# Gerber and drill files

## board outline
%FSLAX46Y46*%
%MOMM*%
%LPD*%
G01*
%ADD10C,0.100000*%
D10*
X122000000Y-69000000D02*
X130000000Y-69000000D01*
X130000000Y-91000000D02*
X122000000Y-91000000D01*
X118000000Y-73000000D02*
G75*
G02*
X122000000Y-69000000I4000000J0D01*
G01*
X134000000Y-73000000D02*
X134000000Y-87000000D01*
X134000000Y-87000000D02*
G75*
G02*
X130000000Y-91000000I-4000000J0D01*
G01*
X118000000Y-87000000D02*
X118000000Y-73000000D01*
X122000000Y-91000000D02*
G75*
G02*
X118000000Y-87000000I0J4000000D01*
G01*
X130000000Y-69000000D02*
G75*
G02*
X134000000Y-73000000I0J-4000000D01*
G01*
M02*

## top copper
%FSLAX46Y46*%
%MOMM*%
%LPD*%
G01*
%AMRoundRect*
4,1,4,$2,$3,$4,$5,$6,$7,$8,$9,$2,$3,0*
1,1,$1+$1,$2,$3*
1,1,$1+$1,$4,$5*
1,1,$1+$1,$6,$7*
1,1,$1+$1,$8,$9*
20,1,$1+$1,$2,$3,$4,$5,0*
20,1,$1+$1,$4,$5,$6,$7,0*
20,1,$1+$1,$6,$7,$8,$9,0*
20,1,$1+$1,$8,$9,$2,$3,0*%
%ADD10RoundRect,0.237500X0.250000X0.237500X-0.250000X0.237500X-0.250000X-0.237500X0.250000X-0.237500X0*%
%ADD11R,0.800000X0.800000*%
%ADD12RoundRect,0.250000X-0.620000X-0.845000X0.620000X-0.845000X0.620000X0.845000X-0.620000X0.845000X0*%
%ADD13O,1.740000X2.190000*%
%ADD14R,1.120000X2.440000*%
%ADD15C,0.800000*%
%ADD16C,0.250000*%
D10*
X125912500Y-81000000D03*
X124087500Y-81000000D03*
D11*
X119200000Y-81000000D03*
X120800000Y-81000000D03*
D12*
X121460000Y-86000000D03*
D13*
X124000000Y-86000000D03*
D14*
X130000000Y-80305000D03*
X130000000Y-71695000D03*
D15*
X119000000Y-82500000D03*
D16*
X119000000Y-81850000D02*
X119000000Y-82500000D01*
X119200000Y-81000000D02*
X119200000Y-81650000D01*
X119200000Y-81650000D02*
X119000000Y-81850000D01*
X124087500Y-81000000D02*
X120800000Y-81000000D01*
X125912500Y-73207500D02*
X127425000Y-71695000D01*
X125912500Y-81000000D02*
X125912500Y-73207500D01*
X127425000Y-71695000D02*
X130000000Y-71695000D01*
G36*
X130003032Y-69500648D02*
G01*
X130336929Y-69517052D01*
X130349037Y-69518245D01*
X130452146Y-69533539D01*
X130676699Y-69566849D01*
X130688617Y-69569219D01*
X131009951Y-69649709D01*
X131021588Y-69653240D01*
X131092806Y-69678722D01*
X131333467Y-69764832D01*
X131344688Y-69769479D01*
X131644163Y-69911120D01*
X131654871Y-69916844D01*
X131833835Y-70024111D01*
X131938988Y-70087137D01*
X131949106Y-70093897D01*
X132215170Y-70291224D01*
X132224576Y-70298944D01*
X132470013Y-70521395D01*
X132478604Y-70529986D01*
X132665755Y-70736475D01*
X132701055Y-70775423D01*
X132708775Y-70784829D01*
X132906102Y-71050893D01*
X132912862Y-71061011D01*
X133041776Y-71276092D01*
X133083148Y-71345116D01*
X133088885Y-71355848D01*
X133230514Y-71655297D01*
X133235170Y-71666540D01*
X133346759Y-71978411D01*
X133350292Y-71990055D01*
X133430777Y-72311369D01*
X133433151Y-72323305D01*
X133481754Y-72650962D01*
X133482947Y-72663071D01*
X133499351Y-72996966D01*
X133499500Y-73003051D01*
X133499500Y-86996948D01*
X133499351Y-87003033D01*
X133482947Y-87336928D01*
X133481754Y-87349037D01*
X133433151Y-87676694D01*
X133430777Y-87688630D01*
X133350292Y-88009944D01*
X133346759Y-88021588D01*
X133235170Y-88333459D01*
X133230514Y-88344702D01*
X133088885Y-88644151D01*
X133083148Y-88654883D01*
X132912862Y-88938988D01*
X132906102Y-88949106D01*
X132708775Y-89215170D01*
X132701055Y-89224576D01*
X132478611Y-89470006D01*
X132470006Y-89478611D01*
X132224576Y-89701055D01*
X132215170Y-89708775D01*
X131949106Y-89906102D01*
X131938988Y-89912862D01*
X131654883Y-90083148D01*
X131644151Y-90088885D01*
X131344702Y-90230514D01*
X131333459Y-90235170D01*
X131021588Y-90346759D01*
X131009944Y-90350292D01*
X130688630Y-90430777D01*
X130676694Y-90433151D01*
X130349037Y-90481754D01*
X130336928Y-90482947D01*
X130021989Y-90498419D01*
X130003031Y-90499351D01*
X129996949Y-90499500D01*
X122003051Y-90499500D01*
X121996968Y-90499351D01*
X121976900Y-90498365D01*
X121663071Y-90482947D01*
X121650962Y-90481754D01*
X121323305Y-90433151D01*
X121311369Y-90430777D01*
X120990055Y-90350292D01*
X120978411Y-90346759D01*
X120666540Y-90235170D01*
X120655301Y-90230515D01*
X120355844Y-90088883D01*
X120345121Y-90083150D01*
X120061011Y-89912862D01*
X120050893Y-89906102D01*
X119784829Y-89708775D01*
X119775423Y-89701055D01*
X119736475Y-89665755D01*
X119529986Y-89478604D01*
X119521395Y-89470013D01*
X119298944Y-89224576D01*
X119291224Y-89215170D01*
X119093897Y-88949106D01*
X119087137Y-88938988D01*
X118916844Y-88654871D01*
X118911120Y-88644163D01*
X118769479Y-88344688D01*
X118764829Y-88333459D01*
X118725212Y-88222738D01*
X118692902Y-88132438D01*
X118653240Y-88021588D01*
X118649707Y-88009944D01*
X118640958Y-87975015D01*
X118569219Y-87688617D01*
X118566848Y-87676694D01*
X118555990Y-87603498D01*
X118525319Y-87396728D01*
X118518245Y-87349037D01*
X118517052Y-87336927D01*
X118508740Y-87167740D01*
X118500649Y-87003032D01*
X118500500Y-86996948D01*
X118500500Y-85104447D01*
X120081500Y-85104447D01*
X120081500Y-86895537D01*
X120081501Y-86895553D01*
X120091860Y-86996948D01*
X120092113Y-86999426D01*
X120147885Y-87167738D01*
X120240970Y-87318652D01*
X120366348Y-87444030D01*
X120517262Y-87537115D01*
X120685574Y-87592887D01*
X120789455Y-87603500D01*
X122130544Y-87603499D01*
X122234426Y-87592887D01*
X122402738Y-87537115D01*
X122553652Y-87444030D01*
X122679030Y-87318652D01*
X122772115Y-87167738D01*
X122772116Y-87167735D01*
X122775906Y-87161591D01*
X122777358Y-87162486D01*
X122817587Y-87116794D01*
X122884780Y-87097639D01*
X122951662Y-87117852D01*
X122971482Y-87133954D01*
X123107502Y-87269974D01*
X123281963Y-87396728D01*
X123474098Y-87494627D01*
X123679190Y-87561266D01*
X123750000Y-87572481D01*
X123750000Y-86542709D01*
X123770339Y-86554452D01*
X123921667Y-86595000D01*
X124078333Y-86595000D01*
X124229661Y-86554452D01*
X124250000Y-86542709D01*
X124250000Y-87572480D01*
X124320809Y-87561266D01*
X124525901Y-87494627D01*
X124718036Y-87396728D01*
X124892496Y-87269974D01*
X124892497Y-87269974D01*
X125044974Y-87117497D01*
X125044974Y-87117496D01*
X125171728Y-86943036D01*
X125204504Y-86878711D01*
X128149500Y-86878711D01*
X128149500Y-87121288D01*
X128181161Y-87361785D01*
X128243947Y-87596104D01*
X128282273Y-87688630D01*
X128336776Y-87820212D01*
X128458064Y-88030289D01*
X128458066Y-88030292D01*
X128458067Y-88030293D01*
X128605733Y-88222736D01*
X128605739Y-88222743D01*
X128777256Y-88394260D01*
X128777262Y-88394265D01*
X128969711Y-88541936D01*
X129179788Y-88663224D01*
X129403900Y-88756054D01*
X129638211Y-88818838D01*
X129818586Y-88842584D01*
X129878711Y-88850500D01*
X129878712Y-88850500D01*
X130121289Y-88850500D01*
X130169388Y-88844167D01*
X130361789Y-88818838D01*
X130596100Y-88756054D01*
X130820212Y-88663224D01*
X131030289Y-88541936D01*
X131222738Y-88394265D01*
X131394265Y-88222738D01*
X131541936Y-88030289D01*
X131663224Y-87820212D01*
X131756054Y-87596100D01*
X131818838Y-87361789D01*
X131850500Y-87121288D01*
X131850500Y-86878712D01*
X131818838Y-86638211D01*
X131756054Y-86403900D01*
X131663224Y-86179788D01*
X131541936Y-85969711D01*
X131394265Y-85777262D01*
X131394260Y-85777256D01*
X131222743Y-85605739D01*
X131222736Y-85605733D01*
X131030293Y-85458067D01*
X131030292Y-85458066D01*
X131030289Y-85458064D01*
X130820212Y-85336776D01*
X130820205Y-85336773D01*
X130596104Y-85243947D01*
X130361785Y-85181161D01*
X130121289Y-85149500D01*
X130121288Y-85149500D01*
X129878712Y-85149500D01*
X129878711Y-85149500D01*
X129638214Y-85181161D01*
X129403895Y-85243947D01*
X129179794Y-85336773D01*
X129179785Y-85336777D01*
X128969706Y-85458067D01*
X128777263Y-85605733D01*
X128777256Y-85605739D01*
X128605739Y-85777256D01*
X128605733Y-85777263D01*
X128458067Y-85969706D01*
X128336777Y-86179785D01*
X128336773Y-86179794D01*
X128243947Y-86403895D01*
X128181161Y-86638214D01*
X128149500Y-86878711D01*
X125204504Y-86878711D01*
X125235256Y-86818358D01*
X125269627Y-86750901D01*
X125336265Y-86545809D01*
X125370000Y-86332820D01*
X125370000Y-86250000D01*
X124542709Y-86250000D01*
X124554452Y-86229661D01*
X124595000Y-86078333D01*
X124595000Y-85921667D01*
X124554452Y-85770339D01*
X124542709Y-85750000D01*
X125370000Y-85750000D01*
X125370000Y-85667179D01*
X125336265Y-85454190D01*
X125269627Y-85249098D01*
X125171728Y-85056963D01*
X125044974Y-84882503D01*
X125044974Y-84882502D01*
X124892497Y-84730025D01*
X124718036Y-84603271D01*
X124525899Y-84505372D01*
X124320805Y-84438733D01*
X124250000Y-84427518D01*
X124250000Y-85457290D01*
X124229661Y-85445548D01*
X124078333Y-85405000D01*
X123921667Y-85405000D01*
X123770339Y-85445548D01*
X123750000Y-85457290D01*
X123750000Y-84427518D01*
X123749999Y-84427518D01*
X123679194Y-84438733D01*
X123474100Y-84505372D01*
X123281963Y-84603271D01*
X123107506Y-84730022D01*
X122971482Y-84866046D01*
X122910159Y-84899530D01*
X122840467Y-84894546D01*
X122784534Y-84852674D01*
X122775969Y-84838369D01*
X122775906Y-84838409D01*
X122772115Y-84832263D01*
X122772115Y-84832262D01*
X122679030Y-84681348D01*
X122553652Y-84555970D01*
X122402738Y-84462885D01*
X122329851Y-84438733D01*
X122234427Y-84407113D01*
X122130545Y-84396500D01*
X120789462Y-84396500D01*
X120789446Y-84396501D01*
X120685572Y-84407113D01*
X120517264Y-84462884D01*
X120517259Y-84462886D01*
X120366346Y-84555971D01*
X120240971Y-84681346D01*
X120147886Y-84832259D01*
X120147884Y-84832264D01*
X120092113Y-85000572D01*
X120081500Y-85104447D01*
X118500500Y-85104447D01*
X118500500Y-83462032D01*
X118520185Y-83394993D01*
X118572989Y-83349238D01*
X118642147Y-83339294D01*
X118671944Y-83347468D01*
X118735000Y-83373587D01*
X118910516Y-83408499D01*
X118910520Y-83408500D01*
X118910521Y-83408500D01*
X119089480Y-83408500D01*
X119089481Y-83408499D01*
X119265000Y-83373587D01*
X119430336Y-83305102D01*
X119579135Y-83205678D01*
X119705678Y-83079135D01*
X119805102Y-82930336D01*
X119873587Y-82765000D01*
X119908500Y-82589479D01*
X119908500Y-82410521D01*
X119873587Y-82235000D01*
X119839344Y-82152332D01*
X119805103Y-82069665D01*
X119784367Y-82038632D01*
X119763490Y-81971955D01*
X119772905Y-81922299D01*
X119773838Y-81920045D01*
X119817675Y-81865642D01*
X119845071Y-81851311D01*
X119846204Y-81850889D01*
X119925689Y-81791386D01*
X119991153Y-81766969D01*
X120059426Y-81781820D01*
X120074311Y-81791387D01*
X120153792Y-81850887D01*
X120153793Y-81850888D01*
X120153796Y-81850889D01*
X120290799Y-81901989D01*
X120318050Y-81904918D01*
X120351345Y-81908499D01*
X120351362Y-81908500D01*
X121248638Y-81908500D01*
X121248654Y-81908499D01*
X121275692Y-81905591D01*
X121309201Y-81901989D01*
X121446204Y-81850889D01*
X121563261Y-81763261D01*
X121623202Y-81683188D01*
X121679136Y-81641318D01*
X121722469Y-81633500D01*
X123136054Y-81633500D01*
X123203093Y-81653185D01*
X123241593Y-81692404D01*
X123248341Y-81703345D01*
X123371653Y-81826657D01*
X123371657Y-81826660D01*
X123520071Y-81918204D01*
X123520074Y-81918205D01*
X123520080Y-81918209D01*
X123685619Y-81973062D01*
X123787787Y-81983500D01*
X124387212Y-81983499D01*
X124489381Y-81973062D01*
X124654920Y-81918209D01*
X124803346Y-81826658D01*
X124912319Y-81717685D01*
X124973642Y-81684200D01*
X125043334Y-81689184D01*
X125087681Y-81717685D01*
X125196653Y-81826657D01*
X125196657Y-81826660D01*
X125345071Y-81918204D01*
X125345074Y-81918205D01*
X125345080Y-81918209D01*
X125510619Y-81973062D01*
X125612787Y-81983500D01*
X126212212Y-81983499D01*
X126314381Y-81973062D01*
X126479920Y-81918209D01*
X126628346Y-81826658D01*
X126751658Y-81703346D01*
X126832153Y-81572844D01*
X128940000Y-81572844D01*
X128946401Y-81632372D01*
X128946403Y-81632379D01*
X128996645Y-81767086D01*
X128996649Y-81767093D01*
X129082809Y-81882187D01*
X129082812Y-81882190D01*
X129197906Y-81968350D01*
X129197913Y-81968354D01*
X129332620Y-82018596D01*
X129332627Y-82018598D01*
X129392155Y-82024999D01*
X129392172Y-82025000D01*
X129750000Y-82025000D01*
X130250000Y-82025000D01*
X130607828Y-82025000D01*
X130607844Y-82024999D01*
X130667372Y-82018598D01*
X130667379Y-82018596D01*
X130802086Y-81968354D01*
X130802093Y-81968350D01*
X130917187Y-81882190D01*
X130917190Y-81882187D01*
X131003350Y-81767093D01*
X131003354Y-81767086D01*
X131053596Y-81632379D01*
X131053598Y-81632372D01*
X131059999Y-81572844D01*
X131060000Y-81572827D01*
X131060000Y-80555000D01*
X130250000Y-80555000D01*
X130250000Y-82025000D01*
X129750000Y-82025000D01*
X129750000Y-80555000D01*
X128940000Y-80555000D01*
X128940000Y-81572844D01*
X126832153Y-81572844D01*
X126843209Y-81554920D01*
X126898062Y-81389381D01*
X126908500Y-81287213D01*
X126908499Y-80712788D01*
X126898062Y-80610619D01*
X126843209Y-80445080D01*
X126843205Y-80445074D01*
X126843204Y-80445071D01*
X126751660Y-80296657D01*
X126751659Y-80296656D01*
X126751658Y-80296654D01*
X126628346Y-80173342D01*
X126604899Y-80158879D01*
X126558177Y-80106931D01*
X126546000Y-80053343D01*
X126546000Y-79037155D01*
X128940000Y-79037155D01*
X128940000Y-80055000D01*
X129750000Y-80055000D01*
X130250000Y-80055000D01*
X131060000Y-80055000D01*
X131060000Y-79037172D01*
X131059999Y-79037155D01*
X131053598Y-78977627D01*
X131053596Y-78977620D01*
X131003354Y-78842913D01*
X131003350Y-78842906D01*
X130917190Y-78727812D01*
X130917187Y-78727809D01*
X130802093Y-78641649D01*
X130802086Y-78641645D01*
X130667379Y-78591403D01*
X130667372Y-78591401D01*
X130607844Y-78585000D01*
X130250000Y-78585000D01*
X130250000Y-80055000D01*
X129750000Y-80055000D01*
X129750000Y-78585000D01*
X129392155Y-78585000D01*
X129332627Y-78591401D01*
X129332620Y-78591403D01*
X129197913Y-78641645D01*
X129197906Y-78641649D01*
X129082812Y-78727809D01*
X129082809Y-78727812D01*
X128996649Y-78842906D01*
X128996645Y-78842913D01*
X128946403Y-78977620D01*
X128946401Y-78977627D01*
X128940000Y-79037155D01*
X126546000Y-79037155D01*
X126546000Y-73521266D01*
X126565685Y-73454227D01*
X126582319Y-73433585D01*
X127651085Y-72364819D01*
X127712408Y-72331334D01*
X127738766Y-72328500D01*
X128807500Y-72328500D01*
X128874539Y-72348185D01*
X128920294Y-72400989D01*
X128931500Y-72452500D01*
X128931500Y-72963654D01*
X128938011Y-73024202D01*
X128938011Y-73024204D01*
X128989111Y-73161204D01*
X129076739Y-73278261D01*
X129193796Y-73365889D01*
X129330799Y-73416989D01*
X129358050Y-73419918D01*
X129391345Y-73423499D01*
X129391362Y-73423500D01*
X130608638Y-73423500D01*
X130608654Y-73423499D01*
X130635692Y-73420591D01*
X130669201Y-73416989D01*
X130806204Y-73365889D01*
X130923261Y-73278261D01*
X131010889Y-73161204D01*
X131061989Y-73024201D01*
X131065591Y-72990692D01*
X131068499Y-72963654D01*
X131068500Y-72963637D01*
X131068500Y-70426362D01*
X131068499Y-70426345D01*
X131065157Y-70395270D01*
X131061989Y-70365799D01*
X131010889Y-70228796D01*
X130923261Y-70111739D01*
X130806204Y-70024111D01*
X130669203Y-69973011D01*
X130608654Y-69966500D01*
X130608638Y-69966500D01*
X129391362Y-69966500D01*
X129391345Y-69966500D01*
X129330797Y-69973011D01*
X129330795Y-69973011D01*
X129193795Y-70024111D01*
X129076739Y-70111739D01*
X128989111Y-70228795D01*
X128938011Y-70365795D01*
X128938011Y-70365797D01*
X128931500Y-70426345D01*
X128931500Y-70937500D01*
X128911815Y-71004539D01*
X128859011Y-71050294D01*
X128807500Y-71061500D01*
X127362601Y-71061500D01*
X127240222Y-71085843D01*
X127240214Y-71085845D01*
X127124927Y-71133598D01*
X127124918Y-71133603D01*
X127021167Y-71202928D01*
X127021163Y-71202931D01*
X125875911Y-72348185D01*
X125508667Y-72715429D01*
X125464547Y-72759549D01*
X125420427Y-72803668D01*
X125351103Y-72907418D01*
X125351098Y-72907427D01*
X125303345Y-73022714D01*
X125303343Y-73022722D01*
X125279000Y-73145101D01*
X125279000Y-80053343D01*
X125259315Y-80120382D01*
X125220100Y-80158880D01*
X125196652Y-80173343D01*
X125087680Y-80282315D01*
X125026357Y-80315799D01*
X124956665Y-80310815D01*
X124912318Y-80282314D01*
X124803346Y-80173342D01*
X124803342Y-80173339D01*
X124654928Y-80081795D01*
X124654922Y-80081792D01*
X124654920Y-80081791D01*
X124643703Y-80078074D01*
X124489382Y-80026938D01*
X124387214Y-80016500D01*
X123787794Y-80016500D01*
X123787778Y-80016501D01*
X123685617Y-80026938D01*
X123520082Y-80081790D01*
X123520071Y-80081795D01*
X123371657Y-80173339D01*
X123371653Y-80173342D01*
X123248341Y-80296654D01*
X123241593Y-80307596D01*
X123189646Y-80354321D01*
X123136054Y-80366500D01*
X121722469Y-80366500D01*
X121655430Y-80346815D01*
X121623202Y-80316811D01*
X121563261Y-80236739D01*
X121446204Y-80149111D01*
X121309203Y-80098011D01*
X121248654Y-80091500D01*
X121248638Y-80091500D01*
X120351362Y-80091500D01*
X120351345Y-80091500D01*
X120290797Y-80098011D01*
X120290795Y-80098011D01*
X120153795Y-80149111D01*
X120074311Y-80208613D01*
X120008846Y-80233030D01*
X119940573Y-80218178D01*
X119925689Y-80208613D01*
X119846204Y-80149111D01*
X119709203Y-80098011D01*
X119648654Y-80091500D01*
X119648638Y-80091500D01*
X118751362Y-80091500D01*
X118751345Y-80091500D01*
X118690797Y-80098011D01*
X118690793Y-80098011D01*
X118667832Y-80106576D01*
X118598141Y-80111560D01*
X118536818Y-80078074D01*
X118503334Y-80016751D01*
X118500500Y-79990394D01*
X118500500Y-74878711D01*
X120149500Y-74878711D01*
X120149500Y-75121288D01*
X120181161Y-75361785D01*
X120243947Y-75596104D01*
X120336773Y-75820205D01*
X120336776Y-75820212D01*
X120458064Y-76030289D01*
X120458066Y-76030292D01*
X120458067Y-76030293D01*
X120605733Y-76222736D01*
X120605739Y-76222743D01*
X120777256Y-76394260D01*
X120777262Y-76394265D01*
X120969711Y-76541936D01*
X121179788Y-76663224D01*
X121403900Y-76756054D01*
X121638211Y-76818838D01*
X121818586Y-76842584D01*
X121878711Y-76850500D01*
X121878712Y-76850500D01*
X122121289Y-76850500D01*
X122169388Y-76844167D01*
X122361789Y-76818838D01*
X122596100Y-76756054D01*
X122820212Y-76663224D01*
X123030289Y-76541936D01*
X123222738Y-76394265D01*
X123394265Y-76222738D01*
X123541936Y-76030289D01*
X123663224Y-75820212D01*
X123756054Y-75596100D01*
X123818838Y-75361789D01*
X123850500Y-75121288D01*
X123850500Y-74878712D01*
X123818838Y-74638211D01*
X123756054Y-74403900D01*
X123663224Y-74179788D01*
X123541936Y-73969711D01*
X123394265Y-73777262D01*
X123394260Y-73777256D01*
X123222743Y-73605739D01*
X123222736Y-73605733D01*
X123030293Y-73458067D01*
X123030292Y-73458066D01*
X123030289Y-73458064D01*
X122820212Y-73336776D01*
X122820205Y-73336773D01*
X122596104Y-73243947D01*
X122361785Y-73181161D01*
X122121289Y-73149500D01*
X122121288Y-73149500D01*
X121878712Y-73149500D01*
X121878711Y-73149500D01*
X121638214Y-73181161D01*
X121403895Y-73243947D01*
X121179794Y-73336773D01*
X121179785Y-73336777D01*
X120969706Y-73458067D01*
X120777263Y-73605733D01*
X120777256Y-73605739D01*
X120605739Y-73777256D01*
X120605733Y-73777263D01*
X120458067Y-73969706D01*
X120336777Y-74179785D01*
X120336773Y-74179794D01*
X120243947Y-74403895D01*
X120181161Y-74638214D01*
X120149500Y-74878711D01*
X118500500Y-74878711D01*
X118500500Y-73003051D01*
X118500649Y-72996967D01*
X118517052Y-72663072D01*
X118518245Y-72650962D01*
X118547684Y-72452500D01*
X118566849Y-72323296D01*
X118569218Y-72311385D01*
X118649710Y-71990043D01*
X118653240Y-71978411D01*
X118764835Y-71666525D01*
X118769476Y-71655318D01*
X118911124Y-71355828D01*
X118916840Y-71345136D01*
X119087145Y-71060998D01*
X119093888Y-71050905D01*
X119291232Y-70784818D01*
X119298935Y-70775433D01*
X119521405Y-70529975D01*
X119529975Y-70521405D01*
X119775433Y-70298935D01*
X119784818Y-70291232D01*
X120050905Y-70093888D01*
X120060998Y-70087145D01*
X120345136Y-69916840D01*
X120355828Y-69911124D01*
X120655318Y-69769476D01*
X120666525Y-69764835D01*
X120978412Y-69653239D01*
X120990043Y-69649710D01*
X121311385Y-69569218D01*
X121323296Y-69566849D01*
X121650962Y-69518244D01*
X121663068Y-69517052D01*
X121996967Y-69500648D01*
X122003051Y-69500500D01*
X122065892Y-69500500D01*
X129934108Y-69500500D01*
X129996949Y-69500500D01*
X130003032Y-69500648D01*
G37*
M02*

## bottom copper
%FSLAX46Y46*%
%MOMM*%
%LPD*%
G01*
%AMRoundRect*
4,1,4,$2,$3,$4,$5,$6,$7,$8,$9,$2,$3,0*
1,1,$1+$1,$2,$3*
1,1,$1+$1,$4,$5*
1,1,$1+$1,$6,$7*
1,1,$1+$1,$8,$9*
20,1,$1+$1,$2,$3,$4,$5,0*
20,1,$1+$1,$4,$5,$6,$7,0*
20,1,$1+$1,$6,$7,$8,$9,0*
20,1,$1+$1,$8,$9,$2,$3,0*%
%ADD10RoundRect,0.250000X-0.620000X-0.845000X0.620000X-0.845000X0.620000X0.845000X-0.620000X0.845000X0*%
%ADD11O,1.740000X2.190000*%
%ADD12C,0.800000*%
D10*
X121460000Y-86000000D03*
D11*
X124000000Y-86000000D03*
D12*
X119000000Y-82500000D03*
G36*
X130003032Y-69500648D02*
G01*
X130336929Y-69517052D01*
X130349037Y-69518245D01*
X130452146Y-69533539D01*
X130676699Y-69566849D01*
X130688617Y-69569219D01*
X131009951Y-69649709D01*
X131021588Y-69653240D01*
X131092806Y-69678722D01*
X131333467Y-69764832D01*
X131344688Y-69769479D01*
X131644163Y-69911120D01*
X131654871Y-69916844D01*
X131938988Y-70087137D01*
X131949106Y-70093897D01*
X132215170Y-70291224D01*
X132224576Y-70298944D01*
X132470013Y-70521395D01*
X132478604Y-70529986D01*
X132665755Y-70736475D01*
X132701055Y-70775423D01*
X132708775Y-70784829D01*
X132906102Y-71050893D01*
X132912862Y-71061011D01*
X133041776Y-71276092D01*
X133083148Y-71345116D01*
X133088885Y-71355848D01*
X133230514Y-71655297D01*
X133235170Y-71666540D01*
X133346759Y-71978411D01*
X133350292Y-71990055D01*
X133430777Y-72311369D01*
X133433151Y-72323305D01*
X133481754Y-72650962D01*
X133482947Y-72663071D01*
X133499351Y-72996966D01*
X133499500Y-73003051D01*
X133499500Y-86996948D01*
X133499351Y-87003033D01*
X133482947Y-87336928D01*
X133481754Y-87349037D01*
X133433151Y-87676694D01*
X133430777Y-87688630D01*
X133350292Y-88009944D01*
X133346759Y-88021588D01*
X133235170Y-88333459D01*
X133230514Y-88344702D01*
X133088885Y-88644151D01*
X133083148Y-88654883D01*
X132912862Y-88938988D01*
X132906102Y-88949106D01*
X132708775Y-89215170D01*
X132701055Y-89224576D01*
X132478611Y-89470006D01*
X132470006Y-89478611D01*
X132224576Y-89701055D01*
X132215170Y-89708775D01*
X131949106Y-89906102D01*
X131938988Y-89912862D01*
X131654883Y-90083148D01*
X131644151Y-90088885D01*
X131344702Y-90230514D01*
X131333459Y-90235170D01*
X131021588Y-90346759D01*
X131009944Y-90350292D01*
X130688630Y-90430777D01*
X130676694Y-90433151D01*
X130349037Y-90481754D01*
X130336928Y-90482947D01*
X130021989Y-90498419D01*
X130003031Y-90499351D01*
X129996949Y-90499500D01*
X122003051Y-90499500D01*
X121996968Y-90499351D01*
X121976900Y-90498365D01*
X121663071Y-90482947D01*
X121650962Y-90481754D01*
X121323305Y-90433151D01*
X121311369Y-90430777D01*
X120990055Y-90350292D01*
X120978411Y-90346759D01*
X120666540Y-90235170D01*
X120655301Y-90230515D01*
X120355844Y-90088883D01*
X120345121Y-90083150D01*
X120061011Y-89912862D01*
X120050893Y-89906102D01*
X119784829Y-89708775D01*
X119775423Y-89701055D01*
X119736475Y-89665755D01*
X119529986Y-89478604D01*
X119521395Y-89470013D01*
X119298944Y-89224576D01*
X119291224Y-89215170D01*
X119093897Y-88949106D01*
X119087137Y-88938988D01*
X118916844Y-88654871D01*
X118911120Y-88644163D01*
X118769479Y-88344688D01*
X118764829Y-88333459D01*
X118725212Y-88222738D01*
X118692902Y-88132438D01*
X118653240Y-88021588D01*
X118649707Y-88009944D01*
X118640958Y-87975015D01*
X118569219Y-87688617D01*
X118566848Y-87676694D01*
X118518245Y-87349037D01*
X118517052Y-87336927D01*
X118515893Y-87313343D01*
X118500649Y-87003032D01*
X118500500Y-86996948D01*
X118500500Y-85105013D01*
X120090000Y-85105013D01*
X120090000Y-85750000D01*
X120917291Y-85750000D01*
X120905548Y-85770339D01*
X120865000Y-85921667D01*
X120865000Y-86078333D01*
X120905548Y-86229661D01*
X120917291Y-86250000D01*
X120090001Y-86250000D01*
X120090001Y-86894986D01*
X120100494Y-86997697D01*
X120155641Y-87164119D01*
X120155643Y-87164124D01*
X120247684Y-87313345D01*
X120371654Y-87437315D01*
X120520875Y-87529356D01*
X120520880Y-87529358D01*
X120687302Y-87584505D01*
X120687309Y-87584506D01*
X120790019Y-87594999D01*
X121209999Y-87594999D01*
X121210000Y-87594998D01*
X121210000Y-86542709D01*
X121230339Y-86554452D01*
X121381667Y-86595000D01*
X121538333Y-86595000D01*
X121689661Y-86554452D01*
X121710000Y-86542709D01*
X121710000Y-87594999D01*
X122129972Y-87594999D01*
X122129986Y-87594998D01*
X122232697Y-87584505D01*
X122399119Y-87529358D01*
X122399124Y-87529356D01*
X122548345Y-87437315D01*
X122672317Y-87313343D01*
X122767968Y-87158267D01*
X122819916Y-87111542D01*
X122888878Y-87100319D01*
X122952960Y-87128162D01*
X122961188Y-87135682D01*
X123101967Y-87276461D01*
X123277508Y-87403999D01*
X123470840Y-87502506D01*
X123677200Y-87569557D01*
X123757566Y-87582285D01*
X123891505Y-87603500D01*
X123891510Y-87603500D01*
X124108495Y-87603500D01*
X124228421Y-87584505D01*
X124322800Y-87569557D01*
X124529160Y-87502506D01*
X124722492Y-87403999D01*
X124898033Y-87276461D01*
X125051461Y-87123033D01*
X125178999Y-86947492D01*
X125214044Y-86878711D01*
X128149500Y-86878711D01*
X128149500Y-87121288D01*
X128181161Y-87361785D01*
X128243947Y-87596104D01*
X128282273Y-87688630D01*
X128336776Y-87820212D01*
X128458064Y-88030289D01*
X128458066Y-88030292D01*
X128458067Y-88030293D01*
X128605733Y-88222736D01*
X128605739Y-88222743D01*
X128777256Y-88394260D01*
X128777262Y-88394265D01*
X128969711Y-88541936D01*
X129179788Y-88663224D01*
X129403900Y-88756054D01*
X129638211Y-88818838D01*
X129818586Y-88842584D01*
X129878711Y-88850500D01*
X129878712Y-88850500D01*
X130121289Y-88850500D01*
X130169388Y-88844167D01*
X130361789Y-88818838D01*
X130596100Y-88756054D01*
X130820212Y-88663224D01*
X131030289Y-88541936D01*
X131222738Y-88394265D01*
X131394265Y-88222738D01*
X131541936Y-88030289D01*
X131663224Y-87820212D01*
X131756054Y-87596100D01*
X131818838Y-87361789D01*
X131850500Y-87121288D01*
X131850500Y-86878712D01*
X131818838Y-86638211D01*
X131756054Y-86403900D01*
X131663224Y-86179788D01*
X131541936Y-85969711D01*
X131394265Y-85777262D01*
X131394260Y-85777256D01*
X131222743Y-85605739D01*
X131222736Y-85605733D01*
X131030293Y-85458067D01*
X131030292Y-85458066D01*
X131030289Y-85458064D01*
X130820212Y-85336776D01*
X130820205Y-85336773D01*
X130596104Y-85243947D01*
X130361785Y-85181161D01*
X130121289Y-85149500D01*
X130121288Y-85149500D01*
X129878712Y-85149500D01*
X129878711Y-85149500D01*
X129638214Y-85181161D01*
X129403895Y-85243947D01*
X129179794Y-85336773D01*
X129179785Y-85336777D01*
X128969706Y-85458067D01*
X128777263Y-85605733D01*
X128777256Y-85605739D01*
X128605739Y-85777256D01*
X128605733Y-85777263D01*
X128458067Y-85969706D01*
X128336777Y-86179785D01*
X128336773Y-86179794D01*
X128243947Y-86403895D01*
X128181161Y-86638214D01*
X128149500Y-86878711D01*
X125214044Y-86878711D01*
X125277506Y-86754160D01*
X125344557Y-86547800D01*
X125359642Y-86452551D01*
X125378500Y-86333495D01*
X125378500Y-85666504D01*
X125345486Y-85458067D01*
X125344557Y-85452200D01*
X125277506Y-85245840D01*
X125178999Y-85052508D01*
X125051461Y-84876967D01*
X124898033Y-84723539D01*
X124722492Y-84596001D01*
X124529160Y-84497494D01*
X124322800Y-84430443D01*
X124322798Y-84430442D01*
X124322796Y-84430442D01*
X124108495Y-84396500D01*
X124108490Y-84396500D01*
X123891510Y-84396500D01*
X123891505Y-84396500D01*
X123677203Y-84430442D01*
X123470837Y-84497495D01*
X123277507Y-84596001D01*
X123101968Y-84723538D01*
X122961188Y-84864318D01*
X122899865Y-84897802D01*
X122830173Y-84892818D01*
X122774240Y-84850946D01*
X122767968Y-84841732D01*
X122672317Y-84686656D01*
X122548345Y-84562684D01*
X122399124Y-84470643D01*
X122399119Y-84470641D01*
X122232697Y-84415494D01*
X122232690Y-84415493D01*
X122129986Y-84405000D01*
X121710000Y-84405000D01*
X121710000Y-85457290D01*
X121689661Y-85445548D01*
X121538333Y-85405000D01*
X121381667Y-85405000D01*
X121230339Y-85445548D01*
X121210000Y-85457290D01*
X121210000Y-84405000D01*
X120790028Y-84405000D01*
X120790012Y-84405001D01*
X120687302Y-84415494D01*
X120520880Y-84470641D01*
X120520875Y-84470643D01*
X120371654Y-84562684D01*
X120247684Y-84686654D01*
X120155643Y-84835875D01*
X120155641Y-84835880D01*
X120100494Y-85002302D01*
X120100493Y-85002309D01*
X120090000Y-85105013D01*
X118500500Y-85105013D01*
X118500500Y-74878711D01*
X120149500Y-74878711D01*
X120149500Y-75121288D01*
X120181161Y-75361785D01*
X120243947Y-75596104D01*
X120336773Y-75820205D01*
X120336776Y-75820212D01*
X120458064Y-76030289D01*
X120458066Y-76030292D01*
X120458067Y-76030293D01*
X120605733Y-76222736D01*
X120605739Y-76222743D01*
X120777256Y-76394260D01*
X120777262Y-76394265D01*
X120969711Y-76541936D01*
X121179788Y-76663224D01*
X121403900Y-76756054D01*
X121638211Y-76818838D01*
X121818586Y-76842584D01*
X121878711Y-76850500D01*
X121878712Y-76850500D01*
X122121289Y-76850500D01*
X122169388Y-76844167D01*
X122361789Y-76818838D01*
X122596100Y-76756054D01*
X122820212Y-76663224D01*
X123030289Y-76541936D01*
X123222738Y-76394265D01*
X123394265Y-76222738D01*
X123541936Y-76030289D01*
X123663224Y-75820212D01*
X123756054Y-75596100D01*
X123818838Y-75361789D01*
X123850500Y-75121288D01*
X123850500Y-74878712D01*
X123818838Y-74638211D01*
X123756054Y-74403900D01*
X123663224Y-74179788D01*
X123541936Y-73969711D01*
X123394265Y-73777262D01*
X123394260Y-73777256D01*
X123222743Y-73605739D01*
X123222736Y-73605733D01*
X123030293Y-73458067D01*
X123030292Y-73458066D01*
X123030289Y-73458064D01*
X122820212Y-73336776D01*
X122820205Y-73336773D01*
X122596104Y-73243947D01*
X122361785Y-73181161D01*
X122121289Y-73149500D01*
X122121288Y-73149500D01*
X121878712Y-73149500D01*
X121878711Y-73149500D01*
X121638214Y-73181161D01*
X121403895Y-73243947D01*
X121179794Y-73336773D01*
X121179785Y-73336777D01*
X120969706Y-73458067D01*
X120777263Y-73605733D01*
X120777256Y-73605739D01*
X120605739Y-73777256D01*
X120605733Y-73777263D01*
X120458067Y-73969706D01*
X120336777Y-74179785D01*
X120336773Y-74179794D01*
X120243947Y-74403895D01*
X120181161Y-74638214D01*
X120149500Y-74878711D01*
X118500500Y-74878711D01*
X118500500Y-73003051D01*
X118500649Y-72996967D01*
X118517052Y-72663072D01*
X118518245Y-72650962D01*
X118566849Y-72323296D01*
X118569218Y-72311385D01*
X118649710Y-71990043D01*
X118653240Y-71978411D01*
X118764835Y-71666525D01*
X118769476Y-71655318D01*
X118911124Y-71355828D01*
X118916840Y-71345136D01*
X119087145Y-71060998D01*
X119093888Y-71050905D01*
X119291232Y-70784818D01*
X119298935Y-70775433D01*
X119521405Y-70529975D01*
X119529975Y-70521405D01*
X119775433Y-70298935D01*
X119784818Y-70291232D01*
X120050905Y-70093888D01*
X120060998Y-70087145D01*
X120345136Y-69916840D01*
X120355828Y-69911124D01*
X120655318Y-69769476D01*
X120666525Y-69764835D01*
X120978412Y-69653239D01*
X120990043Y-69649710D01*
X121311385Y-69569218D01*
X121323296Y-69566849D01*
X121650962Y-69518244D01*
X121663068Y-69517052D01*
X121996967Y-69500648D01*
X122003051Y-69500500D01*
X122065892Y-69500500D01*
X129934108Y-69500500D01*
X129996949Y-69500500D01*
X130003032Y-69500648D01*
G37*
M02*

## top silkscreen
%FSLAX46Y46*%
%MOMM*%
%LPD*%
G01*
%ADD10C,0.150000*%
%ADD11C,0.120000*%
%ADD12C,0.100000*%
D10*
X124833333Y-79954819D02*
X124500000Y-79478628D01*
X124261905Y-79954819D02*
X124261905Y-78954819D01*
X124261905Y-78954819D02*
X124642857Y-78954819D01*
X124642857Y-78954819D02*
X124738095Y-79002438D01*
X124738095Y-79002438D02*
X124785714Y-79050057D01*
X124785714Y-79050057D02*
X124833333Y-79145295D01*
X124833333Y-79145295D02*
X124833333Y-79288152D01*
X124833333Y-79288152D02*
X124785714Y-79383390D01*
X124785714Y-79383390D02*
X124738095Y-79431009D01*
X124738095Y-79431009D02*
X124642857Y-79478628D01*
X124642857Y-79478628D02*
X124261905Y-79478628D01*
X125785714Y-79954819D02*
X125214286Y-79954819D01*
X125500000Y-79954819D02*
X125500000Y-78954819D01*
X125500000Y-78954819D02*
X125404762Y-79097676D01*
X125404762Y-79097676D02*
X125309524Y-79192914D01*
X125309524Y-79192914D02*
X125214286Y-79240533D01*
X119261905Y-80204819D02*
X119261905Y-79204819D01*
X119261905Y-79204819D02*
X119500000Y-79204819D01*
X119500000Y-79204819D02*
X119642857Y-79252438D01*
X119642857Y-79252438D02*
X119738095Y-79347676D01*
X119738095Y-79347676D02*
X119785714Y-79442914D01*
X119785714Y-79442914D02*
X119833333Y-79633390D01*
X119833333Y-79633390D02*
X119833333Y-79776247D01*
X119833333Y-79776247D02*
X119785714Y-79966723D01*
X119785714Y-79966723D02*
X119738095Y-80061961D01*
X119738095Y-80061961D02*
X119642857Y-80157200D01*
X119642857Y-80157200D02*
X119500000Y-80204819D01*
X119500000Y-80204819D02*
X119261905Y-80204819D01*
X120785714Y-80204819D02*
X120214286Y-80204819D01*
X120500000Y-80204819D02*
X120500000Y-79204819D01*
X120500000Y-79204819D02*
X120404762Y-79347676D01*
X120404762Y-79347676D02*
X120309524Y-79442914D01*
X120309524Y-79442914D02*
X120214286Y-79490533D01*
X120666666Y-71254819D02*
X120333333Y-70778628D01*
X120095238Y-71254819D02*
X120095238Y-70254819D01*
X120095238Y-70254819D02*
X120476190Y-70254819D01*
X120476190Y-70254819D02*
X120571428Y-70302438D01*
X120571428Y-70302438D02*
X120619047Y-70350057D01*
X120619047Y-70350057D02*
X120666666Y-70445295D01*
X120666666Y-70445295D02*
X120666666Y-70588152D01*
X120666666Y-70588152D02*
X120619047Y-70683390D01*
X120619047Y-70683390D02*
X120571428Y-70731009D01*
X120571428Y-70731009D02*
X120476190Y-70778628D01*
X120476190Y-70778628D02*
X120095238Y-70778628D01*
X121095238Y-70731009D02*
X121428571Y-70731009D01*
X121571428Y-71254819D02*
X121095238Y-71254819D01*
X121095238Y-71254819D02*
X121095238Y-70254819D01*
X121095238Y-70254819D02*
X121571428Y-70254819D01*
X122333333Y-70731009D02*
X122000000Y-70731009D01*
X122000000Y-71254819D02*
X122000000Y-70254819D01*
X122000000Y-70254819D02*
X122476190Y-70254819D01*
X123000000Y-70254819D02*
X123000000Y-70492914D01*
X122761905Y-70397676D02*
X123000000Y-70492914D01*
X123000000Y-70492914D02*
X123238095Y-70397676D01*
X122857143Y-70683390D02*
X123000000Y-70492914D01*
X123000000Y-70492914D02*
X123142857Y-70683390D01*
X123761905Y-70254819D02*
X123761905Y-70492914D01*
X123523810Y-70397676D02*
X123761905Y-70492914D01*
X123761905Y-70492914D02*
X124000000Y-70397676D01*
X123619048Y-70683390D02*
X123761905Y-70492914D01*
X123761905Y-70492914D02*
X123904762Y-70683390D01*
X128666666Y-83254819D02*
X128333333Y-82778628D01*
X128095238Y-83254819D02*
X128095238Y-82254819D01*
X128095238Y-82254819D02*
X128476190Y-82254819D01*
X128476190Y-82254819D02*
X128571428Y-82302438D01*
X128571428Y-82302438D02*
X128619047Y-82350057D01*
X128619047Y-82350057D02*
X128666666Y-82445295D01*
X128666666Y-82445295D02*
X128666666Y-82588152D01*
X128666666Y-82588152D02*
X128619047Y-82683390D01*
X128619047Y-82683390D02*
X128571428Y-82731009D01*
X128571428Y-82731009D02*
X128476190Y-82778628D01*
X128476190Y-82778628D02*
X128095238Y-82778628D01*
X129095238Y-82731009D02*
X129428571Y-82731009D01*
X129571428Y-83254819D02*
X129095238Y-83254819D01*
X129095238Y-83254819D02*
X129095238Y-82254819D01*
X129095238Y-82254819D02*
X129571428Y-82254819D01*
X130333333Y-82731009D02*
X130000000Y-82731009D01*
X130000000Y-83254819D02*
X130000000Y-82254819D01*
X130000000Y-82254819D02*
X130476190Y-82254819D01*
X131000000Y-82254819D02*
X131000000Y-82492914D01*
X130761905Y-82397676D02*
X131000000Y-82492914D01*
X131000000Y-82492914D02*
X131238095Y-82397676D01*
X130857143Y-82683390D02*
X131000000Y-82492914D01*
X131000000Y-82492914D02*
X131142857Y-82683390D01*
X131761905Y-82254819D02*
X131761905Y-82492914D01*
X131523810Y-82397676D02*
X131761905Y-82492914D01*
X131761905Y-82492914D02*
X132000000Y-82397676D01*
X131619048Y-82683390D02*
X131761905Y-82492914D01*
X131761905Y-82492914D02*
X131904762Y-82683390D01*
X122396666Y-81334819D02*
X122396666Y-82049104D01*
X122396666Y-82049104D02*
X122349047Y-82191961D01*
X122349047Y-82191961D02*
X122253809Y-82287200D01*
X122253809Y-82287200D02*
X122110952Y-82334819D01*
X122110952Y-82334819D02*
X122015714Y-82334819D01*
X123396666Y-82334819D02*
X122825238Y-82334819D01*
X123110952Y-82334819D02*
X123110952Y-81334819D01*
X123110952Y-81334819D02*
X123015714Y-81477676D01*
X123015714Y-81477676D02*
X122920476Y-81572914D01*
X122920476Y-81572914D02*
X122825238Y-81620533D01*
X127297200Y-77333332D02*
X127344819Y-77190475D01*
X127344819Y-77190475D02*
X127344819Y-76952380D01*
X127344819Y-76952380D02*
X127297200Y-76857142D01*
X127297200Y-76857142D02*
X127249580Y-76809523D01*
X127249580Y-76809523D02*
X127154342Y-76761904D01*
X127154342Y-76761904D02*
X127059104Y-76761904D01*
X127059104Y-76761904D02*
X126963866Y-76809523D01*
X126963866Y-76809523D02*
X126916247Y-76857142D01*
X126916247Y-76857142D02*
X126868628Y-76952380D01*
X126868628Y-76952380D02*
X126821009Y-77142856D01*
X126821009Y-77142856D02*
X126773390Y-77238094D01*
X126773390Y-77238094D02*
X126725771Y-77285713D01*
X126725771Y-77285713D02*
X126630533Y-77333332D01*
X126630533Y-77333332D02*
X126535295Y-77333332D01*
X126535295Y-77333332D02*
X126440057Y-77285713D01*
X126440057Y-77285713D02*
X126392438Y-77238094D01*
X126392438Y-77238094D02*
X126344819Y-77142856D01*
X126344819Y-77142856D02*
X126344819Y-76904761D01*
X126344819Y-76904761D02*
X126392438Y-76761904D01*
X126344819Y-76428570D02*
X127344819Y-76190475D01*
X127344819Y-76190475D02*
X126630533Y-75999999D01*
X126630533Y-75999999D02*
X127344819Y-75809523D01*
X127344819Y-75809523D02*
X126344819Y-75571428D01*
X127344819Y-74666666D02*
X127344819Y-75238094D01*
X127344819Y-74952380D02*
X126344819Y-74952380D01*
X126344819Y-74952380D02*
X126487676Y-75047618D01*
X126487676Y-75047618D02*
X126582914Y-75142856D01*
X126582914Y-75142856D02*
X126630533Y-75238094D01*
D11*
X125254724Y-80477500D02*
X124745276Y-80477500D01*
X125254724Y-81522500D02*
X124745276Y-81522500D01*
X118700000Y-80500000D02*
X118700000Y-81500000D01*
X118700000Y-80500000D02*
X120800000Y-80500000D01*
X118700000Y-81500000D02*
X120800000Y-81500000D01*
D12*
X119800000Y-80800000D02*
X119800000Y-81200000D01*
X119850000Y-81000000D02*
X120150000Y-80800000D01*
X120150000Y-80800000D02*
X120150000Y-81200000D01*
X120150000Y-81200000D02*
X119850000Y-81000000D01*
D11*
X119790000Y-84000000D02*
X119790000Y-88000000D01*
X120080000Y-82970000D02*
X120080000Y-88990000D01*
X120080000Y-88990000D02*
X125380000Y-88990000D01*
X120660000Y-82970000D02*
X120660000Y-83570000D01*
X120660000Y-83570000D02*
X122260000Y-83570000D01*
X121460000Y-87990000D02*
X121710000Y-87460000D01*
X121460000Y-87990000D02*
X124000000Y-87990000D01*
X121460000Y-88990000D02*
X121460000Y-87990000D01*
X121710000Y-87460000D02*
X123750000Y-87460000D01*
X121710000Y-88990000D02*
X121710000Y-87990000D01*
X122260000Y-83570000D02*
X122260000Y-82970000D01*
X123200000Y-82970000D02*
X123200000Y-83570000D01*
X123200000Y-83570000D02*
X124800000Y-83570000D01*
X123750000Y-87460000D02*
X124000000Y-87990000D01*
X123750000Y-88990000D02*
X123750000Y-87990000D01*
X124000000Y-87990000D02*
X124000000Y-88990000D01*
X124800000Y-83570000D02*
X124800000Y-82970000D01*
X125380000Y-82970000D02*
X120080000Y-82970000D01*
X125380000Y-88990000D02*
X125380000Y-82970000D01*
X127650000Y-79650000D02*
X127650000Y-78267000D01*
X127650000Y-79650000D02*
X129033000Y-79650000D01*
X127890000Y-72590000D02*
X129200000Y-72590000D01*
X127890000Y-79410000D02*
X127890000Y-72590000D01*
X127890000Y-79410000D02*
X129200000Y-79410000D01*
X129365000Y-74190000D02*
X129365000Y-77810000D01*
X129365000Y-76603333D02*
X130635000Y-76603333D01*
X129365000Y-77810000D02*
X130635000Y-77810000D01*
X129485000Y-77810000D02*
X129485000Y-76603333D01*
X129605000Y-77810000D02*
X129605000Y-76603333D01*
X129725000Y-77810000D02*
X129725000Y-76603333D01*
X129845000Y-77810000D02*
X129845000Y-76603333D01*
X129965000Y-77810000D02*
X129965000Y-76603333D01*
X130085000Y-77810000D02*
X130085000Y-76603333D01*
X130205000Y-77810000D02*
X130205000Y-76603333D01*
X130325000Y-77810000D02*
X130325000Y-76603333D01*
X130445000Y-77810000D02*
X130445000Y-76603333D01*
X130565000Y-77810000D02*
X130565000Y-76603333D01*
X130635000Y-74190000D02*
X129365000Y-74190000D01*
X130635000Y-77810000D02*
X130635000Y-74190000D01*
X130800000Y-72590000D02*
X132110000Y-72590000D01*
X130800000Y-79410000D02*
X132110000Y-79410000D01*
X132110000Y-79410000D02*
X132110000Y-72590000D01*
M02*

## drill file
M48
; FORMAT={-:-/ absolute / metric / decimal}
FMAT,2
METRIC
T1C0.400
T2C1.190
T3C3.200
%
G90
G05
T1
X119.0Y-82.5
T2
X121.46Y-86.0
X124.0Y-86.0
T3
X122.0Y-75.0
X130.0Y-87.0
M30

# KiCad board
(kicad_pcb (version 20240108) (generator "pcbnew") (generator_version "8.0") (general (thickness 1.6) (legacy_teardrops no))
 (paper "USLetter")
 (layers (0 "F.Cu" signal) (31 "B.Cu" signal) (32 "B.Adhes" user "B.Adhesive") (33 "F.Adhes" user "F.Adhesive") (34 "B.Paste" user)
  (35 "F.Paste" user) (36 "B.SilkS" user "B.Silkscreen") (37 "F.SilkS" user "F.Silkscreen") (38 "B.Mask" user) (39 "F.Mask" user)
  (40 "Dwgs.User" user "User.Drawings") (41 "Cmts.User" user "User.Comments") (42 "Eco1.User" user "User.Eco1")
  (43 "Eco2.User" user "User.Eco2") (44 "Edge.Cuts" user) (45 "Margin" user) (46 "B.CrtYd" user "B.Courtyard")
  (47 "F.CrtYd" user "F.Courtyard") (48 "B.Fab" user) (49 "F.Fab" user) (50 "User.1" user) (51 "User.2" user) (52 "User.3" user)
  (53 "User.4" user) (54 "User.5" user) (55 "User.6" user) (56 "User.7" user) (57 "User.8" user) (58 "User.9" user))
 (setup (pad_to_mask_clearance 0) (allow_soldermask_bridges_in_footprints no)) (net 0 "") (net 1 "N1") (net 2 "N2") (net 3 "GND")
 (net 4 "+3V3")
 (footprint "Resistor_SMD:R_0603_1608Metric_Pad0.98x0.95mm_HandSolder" (layer "F.Cu") (at 125 81 180)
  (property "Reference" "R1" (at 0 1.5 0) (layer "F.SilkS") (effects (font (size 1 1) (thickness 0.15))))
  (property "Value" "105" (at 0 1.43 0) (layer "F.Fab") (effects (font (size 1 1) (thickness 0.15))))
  (fp_line (start -0.254724 0.5225) (end 0.254724 0.5225) (stroke (width 0.12) (type solid)) (layer "F.SilkS"))
  (fp_line (start -0.254724 -0.5225) (end 0.254724 -0.5225) (stroke (width 0.12) (type solid)) (layer "F.SilkS"))
  (pad "1" smd roundrect (at -0.9125 0 180) (size 0.975 0.95) (layers "F.Cu" "F.Paste" "F.Mask") (roundrect_rratio 0.25) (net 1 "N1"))
  (pad "2" smd roundrect (at 0.9125 0 180) (size 0.975 0.95) (layers "F.Cu" "F.Paste" "F.Mask") (roundrect_rratio 0.25) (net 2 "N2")))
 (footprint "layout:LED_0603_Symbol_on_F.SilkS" (layer "F.Cu") (at 120 81)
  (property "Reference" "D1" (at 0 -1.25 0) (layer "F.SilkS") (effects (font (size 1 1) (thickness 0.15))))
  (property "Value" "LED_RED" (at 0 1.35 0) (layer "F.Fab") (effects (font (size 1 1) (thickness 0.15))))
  (fp_line (start -1.3 -0.5) (end -1.3 0.5) (stroke (width 0.12) (type solid)) (layer "F.SilkS"))
  (fp_line (start -1.3 -0.5) (end 0.8 -0.5) (stroke (width 0.12) (type solid)) (layer "F.SilkS"))
  (fp_line (start -1.3 0.5) (end 0.8 0.5) (stroke (width 0.12) (type solid)) (layer "F.SilkS"))
  (fp_line (start -0.2 -0.2) (end -0.2 0.2) (stroke (width 0.1) (type solid)) (layer "F.SilkS"))
  (fp_line (start -0.15 0) (end 0.15 -0.2) (stroke (width 0.1) (type solid)) (layer "F.SilkS"))
  (fp_line (start 0.15 -0.2) (end 0.15 0.2) (stroke (width 0.1) (type solid)) (layer "F.SilkS"))
  (fp_line (start 0.15 0.2) (end -0.15 0) (stroke (width 0.1) (type solid)) (layer "F.SilkS"))
  (pad "1" smd rect (at -0.8 0 180) (size 0.8 0.8) (layers "F.Cu" "F.Paste" "F.Mask") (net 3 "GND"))
  (pad "2" smd rect (at 0.8 0 180) (size 0.8 0.8) (layers "F.Cu" "F.Paste" "F.Mask") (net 2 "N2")))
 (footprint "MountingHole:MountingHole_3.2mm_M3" (layer "F.Cu") (at 122 75)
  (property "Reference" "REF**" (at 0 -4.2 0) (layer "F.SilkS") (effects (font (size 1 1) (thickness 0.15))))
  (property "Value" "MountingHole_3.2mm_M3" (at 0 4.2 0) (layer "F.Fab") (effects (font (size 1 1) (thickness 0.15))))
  (pad "" np_thru_hole circle (at 0 0) (size 3.2 3.2) (drill 3.2) (layers "*.Cu" "*.Mask")))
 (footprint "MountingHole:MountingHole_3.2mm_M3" (layer "F.Cu") (at 130 87)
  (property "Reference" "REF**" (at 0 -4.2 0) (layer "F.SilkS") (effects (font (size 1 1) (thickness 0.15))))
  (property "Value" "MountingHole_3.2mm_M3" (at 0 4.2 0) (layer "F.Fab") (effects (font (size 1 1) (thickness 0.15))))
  (pad "" np_thru_hole circle (at 0 0) (size 3.2 3.2) (drill 3.2) (layers "*.Cu" "*.Mask")))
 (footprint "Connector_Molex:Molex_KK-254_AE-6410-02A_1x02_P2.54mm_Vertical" (layer "F.Cu") (at 121.46 86)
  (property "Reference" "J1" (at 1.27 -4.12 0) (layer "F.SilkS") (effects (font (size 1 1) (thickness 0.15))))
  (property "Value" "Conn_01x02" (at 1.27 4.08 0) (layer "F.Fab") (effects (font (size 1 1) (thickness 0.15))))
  (fp_line (start -1.67 -2) (end -1.67 2) (stroke (width 0.12) (type solid)) (layer "F.SilkS"))
  (fp_line (start -1.38 -3.03) (end -1.38 2.99) (stroke (width 0.12) (type solid)) (layer "F.SilkS"))
  (fp_line (start -1.38 2.99) (end 3.92 2.99) (stroke (width 0.12) (type solid)) (layer "F.SilkS"))
  (fp_line (start -0.8 -3.03) (end -0.8 -2.43) (stroke (width 0.12) (type solid)) (layer "F.SilkS"))
  (fp_line (start -0.8 -2.43) (end 0.8 -2.43) (stroke (width 0.12) (type solid)) (layer "F.SilkS"))
  (fp_line (start 0 1.99) (end 0.25 1.46) (stroke (width 0.12) (type solid)) (layer "F.SilkS"))
  (fp_line (start 0 1.99) (end 2.54 1.99) (stroke (width 0.12) (type solid)) (layer "F.SilkS"))
  (fp_line (start 0 2.99) (end 0 1.99) (stroke (width 0.12) (type solid)) (layer "F.SilkS"))
  (fp_line (start 0.25 1.46) (end 2.29 1.46) (stroke (width 0.12) (type solid)) (layer "F.SilkS"))
  (fp_line (start 0.25 2.99) (end 0.25 1.99) (stroke (width 0.12) (type solid)) (layer "F.SilkS"))
  (fp_line (start 0.8 -2.43) (end 0.8 -3.03) (stroke (width 0.12) (type solid)) (layer "F.SilkS"))
  (fp_line (start 1.74 -3.03) (end 1.74 -2.43) (stroke (width 0.12) (type solid)) (layer "F.SilkS"))
  (fp_line (start 1.74 -2.43) (end 3.34 -2.43) (stroke (width 0.12) (type solid)) (layer "F.SilkS"))
  (fp_line (start 2.29 1.46) (end 2.54 1.99) (stroke (width 0.12) (type solid)) (layer "F.SilkS"))
  (fp_line (start 2.29 2.99) (end 2.29 1.99) (stroke (width 0.12) (type solid)) (layer "F.SilkS"))
  (fp_line (start 2.54 1.99) (end 2.54 2.99) (stroke (width 0.12) (type solid)) (layer "F.SilkS"))
  (fp_line (start 3.34 -2.43) (end 3.34 -3.03) (stroke (width 0.12) (type solid)) (layer "F.SilkS"))
  (fp_line (start 3.92 -3.03) (end -1.38 -3.03) (stroke (width 0.12) (type solid)) (layer "F.SilkS"))
  (fp_line (start 3.92 2.99) (end 3.92 -3.03) (stroke (width 0.12) (type solid)) (layer "F.SilkS"))
  (pad "1" thru_hole roundrect (at 0 0) (size 1.74 2.19) (drill 1.19) (layers "*.Cu" "*.Mask") (remove_unused_layers no)
   (roundrect_rratio 0.143678) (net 3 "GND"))
  (pad "2" thru_hole oval (at 2.54 0) (size 1.74 2.19) (drill 1.19) (layers "*.Cu" "*.Mask") (remove_unused_layers no) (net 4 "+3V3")))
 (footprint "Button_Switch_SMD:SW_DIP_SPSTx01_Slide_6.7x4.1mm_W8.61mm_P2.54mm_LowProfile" (layer "F.Cu") (at 130 76 90)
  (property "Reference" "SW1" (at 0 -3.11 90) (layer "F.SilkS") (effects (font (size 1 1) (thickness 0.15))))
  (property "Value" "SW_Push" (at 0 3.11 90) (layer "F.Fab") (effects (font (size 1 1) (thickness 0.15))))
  (fp_line (start -3.65 -2.35) (end -2.267 -2.35) (stroke (width 0.12) (type solid)) (layer "F.SilkS"))
  (fp_line (start -3.65 -2.35) (end -3.65 -0.967) (stroke (width 0.12) (type solid)) (layer "F.SilkS"))
  (fp_line (start 3.41 -2.11) (end 3.41 -0.8) (stroke (width 0.12) (type solid)) (layer "F.SilkS"))
  (fp_line (start -3.41 -2.11) (end 3.41 -2.11) (stroke (width 0.12) (type solid)) (layer "F.SilkS"))
  (fp_line (start -3.41 -2.11) (end -3.41 -0.8) (stroke (width 0.12) (type solid)) (layer "F.SilkS"))
  (fp_line (start 1.81 -0.635) (end -1.81 -0.635) (stroke (width 0.12) (type solid)) (layer "F.SilkS"))
  (fp_line (start -0.603333 -0.635) (end -0.603333 0.635) (stroke (width 0.12) (type solid)) (layer "F.SilkS"))
  (fp_line (start -1.81 -0.635) (end -1.81 0.635) (stroke (width 0.12) (type solid)) (layer "F.SilkS"))
  (fp_line (start -1.81 -0.515) (end -0.603333 -0.515) (stroke (width 0.12) (type solid)) (layer "F.SilkS"))
  (fp_line (start -1.81 -0.395) (end -0.603333 -0.395) (stroke (width 0.12) (type solid)) (layer "F.SilkS"))
  (fp_line (start -1.81 -0.275) (end -0.603333 -0.275) (stroke (width 0.12) (type solid)) (layer "F.SilkS"))
  (fp_line (start -1.81 -0.155) (end -0.603333 -0.155) (stroke (width 0.12) (type solid)) (layer "F.SilkS"))
  (fp_line (start -1.81 -0.035) (end -0.603333 -0.035) (stroke (width 0.12) (type solid)) (layer "F.SilkS"))
  (fp_line (start -1.81 0.085) (end -0.603333 0.085) (stroke (width 0.12) (type solid)) (layer "F.SilkS"))
  (fp_line (start -1.81 0.205) (end -0.603333 0.205) (stroke (width 0.12) (type solid)) (layer "F.SilkS"))
  (fp_line (start -1.81 0.325) (end -0.603333 0.325) (stroke (width 0.12) (type solid)) (layer "F.SilkS"))
  (fp_line (start -1.81 0.445) (end -0.603333 0.445) (stroke (width 0.12) (type solid)) (layer "F.SilkS"))
  (fp_line (start -1.81 0.565) (end -0.603333 0.565) (stroke (width 0.12) (type solid)) (layer "F.SilkS"))
  (fp_line (start 1.81 0.635) (end 1.81 -0.635) (stroke (width 0.12) (type solid)) (layer "F.SilkS"))
  (fp_line (start -1.81 0.635) (end 1.81 0.635) (stroke (width 0.12) (type solid)) (layer "F.SilkS"))
  (fp_line (start 3.41 0.8) (end 3.41 2.11) (stroke (width 0.12) (type solid)) (layer "F.SilkS"))
  (fp_line (start -3.41 0.8) (end -3.41 2.11) (stroke (width 0.12) (type solid)) (layer "F.SilkS"))
  (fp_line (start -3.41 2.11) (end 3.41 2.11) (stroke (width 0.12) (type solid)) (layer "F.SilkS"))
  (pad "1" smd rect (at -4.305 0 90) (size 2.44 1.12) (layers "F.Cu" "F.Paste" "F.Mask") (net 4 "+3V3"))
  (pad "2" smd rect (at 4.305 0 90) (size 2.44 1.12) (layers "F.Cu" "F.Paste" "F.Mask") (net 1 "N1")))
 (gr_line (start 122 69) (end 130 69) (stroke (width 0.1) (type default)) (layer "Edge.Cuts"))
 (gr_line (start 130 91) (end 122 91) (stroke (width 0.1) (type default)) (layer "Edge.Cuts"))
 (gr_arc (start 118 73) (mid 119.171573 70.171573) (end 122 69) (stroke (width 0.1) (type default)) (layer "Edge.Cuts"))
 (gr_line (start 134 73) (end 134 87) (stroke (width 0.1) (type default)) (layer "Edge.Cuts"))
 (gr_arc (start 134 87) (mid 132.828427 89.828427) (end 130 91) (stroke (width 0.1) (type default)) (layer "Edge.Cuts"))
 (gr_line (start 118 87) (end 118 73) (stroke (width 0.1) (type default)) (layer "Edge.Cuts"))
 (gr_arc (start 122 91) (mid 119.171573 89.828427) (end 118 87) (stroke (width 0.1) (type default)) (layer "Edge.Cuts"))
 (gr_arc (start 130 69) (mid 132.828427 70.171573) (end 134 73) (stroke (width 0.1) (type default)) (layer "Edge.Cuts"))
 (segment (start 119 81.85) (end 119 82.5) (width 0.25) (layer "F.Cu") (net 3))
 (segment (start 119.2 81) (end 119.2 81.65) (width 0.25) (layer "F.Cu") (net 3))
 (segment (start 119.2 81.65) (end 119 81.85) (width 0.25) (layer "F.Cu") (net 3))
 (via (at 119 82.5) (size 0.8) (drill 0.4) (layers "F.Cu" "B.Cu") (free yes) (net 3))
 (segment (start 124.0875 81) (end 120.8 81) (width 0.25) (layer "F.Cu") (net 2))
 (segment (start 125.9125 73.2075) (end 127.425 71.695) (width 0.25) (layer "F.Cu") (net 1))
 (segment (start 125.9125 81) (end 125.9125 73.2075) (width 0.25) (layer "F.Cu") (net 1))
 (segment (start 127.425 71.695) (end 130 71.695) (width 0.25) (layer "F.Cu") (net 1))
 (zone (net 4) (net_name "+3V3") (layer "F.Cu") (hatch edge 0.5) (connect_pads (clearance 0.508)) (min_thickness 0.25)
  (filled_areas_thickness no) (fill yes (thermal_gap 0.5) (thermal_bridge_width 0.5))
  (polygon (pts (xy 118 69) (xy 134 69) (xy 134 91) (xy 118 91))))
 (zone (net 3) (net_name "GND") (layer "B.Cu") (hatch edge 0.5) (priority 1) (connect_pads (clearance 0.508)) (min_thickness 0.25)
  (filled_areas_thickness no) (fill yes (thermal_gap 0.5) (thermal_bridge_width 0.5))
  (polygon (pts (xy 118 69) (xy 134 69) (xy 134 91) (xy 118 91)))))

